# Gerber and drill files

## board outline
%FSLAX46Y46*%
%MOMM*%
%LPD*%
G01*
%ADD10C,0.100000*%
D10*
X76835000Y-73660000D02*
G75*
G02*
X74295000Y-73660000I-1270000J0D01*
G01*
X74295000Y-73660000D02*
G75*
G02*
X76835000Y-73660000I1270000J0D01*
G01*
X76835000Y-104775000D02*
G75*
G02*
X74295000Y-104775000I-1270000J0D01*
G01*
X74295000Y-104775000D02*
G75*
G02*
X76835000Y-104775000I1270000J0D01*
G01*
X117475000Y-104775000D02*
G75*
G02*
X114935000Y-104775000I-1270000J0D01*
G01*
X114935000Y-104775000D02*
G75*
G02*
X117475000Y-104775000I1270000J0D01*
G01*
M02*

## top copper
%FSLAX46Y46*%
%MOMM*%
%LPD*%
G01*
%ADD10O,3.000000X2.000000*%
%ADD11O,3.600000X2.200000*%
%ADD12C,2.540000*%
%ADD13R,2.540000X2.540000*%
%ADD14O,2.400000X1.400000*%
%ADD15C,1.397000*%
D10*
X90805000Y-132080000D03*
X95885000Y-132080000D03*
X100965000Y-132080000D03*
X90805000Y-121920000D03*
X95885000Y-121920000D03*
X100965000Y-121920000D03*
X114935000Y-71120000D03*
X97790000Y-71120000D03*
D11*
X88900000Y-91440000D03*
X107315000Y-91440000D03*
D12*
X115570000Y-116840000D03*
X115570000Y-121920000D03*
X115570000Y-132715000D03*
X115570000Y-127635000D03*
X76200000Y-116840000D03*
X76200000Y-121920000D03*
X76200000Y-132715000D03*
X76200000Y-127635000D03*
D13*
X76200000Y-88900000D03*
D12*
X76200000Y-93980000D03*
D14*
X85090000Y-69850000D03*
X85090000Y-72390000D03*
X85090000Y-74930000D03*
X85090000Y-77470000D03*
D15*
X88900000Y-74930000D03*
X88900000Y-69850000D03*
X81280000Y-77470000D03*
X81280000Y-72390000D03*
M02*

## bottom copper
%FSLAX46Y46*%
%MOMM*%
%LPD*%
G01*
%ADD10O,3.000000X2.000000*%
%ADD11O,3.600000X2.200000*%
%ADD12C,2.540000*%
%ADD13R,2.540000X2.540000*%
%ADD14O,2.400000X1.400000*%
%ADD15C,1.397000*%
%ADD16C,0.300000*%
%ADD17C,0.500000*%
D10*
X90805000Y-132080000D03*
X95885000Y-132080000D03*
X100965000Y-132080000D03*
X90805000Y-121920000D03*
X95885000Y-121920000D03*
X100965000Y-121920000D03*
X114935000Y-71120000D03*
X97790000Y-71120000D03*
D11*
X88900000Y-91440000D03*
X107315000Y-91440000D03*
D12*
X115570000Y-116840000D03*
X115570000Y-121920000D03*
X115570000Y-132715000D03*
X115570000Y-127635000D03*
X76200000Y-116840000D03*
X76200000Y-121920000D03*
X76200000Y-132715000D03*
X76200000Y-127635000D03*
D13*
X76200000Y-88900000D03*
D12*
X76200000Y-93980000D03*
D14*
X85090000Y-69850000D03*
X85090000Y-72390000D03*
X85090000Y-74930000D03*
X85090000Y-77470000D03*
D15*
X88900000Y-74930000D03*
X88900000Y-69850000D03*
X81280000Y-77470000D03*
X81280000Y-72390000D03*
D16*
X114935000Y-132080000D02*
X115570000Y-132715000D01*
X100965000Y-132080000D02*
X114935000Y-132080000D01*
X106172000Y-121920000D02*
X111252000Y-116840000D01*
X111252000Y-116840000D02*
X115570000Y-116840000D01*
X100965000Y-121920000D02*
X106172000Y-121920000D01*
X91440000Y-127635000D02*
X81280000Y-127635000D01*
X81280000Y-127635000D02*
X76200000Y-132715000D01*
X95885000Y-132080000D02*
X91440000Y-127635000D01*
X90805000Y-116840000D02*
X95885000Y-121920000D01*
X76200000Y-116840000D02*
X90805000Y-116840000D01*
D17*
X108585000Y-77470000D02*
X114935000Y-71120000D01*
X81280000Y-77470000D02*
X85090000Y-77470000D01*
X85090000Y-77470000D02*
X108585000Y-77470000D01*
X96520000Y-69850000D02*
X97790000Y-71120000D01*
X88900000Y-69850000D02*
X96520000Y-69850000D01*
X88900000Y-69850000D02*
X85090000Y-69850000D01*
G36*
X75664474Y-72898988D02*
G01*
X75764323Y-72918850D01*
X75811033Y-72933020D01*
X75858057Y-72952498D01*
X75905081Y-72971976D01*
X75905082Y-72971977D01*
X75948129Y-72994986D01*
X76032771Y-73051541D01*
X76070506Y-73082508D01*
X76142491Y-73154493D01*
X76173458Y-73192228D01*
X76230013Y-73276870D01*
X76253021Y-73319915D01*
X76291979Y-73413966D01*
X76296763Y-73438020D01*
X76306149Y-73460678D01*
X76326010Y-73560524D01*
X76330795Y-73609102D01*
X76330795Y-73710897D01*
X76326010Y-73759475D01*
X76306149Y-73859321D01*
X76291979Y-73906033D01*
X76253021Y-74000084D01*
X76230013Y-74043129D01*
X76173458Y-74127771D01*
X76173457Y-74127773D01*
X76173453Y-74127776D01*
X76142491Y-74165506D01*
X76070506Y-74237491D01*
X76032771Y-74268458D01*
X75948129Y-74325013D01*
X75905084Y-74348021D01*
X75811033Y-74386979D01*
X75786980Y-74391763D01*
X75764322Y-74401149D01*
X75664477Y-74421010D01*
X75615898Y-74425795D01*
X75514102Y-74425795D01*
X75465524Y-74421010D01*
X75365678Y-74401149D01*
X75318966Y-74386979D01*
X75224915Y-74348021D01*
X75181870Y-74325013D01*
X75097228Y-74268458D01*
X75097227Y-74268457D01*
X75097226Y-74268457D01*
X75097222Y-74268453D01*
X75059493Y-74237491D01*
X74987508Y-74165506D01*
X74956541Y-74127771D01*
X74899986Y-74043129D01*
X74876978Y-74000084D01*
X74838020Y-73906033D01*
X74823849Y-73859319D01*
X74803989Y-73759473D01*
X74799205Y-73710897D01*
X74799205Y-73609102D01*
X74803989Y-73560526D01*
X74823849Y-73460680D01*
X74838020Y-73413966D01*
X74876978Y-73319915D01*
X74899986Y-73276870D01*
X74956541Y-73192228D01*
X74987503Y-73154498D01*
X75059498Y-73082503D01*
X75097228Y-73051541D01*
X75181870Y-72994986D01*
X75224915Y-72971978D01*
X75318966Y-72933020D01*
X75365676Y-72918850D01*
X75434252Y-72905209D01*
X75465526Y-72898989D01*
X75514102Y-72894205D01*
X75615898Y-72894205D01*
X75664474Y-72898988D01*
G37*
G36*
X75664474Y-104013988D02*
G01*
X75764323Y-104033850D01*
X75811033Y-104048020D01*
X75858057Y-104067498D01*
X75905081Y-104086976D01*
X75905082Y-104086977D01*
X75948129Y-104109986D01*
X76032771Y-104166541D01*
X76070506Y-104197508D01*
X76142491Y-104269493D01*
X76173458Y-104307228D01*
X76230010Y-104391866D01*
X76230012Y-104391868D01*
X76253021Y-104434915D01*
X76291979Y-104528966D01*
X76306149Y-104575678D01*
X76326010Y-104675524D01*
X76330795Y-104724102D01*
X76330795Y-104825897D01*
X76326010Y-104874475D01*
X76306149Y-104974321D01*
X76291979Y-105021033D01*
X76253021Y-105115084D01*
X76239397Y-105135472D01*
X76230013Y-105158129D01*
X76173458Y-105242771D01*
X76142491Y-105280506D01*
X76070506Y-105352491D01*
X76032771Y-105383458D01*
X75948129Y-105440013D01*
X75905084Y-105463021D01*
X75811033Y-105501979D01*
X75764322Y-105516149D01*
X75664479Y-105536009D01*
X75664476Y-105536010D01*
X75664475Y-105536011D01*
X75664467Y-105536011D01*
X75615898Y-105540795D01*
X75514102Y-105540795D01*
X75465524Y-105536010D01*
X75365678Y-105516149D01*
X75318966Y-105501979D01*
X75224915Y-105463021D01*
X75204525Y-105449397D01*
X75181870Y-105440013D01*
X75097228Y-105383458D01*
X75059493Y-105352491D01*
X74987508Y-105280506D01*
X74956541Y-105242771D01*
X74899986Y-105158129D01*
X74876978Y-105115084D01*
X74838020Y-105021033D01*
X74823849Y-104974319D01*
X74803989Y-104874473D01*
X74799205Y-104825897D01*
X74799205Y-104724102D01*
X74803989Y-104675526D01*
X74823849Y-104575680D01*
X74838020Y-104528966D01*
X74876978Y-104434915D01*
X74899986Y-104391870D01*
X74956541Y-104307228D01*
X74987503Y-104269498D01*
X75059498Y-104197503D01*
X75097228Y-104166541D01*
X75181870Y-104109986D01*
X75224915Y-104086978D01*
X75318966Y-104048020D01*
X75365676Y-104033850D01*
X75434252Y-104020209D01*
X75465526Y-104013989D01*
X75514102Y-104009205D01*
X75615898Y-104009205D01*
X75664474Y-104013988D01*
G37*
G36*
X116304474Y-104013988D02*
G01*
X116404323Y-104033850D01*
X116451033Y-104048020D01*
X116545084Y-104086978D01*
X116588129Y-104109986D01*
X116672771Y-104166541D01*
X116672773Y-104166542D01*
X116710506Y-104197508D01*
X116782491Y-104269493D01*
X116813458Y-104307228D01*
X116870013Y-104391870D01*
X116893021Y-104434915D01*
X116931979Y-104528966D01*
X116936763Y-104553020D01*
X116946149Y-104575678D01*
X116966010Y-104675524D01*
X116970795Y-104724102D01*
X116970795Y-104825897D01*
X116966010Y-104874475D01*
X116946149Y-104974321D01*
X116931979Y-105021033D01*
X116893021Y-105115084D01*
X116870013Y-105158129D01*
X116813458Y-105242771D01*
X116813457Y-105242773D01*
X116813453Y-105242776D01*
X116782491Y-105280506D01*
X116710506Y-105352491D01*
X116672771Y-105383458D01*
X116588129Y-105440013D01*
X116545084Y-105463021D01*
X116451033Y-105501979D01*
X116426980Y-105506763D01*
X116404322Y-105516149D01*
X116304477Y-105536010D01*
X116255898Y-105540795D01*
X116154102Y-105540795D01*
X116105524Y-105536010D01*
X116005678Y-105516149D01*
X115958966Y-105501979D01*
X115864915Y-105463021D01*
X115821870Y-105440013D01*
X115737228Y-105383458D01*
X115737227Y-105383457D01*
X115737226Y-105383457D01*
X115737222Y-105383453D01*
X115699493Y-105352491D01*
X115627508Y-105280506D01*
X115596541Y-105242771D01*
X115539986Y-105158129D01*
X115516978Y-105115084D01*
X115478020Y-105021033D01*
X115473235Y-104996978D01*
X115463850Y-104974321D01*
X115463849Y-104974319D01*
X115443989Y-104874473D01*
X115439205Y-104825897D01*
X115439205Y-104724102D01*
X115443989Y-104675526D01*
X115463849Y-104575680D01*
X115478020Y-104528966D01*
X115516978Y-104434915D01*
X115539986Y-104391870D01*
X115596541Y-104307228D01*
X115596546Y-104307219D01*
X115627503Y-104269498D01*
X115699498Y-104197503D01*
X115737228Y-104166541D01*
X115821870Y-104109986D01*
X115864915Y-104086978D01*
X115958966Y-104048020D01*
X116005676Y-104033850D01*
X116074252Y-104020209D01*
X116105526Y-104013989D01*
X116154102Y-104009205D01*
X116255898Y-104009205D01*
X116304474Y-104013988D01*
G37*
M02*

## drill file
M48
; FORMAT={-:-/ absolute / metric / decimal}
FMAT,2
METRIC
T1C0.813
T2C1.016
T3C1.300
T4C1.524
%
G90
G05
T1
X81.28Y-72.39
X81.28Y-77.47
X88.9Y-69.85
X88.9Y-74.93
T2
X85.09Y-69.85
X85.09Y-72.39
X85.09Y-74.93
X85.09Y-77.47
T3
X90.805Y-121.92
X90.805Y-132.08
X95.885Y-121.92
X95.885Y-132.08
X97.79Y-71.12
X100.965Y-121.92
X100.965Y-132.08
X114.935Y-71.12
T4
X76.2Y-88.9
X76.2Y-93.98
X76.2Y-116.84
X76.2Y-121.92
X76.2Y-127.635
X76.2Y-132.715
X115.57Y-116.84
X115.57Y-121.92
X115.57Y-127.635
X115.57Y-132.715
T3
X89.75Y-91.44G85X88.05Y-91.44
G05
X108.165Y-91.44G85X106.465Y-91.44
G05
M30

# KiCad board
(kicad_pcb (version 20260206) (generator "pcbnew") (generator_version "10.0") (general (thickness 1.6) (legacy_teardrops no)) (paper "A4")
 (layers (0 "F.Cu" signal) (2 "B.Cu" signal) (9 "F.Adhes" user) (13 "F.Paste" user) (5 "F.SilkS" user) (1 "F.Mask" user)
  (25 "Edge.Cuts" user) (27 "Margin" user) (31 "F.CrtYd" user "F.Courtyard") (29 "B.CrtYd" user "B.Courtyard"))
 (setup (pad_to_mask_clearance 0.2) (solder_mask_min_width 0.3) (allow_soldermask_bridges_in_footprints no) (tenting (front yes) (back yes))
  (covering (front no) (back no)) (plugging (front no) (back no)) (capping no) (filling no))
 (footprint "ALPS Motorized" (layer "F.Cu") (at 95.885 96.52 180)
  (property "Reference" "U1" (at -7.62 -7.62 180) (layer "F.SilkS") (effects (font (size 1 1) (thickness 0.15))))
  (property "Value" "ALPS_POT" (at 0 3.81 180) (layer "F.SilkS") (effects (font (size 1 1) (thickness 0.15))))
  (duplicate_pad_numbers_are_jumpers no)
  (pad "1" thru_hole oval (at 5.08 -35.56 180) (size 3 2) (drill 1.3) (layers "*.Cu" "*.Mask" "F.SilkS") (remove_unused_layers no)
   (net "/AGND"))
  (pad "2" thru_hole oval (at 0 -35.56 180) (size 3 2) (drill 1.3) (layers "*.Cu" "*.Mask" "F.SilkS") (remove_unused_layers no)
   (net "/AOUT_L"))
  (pad "3" thru_hole oval (at -5.08 -35.56 180) (size 3 2) (drill 1.3) (layers "*.Cu" "*.Mask" "F.SilkS") (remove_unused_layers no)
   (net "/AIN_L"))
  (pad "4" thru_hole oval (at 5.08 -25.4 180) (size 3 2) (drill 1.3) (layers "*.Cu" "*.Mask" "F.SilkS") (remove_unused_layers no)
   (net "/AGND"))
  (pad "5" thru_hole oval (at 0 -25.4 180) (size 3 2) (drill 1.3) (layers "*.Cu" "*.Mask" "F.SilkS") (remove_unused_layers no)
   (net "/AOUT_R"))
  (pad "6" thru_hole oval (at -5.08 -25.4 180) (size 3 2) (drill 1.3) (layers "*.Cu" "*.Mask" "F.SilkS") (remove_unused_layers no)
   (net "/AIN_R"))
  (pad "7" thru_hole oval (at -19.05 25.4 180) (size 3 2) (drill 1.3) (layers "*.Cu" "*.Mask" "F.SilkS") (remove_unused_layers no)
   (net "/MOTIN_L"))
  (pad "8" thru_hole oval (at -1.905 25.4 180) (size 3 2) (drill 1.3) (layers "*.Cu" "*.Mask" "F.SilkS") (remove_unused_layers no)
   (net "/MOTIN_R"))
  (pad "9" thru_hole oval (at 6.985 5.08 180) (size 3.6 2.2) (drill oval 3 1.3) (layers "*.Cu" "*.Mask" "F.SilkS") (remove_unused_layers no)
   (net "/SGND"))
  (pad "10" thru_hole oval (at -11.43 5.08 180) (size 3.6 2.2) (drill oval 3 1.3) (layers "*.Cu" "*.Mask" "F.SilkS")
   (remove_unused_layers no) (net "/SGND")))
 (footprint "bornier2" (layer "F.Cu") (at 115.57 119.38 -90)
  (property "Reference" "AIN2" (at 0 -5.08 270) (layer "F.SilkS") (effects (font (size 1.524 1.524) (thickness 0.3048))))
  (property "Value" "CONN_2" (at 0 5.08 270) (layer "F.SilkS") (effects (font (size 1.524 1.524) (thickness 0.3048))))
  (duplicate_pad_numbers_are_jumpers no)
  (pad "1" thru_hole circle (at -2.54 0 270) (size 2.54 2.54) (drill 1.524) (layers "*.Cu" "*.Mask" "F.SilkS") (remove_unused_layers no)
   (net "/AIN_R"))
  (pad "2" thru_hole circle (at 2.54 0 270) (size 2.54 2.54) (drill 1.524) (layers "*.Cu" "*.Mask" "F.SilkS") (remove_unused_layers no)
   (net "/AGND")))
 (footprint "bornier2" (layer "F.Cu") (at 115.57 130.175 90)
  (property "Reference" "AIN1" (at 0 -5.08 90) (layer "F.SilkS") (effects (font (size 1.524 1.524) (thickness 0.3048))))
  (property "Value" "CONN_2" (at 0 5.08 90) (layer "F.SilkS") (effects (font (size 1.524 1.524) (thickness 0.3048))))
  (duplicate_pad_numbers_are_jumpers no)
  (pad "1" thru_hole circle (at -2.54 0 90) (size 2.54 2.54) (drill 1.524) (layers "*.Cu" "*.Mask" "F.SilkS") (remove_unused_layers no)
   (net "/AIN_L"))
  (pad "2" thru_hole circle (at 2.54 0 90) (size 2.54 2.54) (drill 1.524) (layers "*.Cu" "*.Mask" "F.SilkS") (remove_unused_layers no)
   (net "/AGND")))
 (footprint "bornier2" (layer "F.Cu") (at 76.2 119.38 -90)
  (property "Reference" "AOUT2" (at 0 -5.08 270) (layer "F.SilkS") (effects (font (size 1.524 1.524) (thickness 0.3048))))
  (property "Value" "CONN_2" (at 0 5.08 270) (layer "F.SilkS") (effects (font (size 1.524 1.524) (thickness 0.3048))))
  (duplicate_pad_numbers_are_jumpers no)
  (pad "1" thru_hole circle (at -2.54 0 270) (size 2.54 2.54) (drill 1.524) (layers "*.Cu" "*.Mask" "F.SilkS") (remove_unused_layers no)
   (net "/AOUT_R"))
  (pad "2" thru_hole circle (at 2.54 0 270) (size 2.54 2.54) (drill 1.524) (layers "*.Cu" "*.Mask" "F.SilkS") (remove_unused_layers no)
   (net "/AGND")))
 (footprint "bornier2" (layer "F.Cu") (at 76.2 130.175 90)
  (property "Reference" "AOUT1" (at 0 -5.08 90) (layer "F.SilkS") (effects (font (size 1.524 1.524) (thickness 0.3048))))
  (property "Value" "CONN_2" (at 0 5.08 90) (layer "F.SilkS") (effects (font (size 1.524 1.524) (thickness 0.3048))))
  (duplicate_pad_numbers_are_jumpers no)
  (pad "1" thru_hole circle (at -2.54 0 90) (size 2.54 2.54) (drill 1.524) (layers "*.Cu" "*.Mask" "F.SilkS") (remove_unused_layers no)
   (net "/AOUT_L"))
  (pad "2" thru_hole circle (at 2.54 0 90) (size 2.54 2.54) (drill 1.524) (layers "*.Cu" "*.Mask" "F.SilkS") (remove_unused_layers no)
   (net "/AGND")))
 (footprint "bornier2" (layer "F.Cu") (at 76.2 91.44 -90)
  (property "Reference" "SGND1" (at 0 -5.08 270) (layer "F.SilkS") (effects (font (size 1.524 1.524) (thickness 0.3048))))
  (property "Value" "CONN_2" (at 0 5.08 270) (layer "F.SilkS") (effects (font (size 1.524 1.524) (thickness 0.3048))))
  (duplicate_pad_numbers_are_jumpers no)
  (pad "1" thru_hole rect (at -2.54 0 270) (size 2.54 2.54) (drill 1.524) (layers "*.Cu" "*.Mask" "F.SilkS") (remove_unused_layers no)
   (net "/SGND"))
  (pad "2" thru_hole circle (at 2.54 0 270) (size 2.54 2.54) (drill 1.524) (layers "*.Cu" "*.Mask" "F.SilkS") (remove_unused_layers no)
   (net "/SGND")))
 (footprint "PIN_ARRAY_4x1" (layer "F.Cu") (at 85.09 73.66 -90)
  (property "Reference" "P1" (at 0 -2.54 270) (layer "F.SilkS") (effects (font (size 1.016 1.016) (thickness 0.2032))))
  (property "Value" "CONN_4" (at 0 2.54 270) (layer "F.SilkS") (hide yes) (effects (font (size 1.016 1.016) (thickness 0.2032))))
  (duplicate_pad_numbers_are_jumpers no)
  (pad "1" thru_hole oval (at -3.81 0 270) (size 1.4 2.4) (drill 1.016) (layers "*.Cu" "*.Mask" "F.SilkS") (remove_unused_layers no)
   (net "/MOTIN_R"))
  (pad "2" thru_hole oval (at -1.27 0 270) (size 1.4 2.4) (drill 1.016) (layers "*.Cu" "*.Mask" "F.SilkS") (remove_unused_layers no)
   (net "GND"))
  (pad "3" thru_hole oval (at 1.27 0 270) (size 1.4 2.4) (drill 1.016) (layers "*.Cu" "*.Mask" "F.SilkS") (remove_unused_layers no)
   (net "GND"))
  (pad "4" thru_hole oval (at 3.81 0 270) (size 1.4 2.4) (drill 1.016) (layers "*.Cu" "*.Mask" "F.SilkS") (remove_unused_layers no)
   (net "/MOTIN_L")))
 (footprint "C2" (layer "F.Cu") (at 88.9 72.39 90)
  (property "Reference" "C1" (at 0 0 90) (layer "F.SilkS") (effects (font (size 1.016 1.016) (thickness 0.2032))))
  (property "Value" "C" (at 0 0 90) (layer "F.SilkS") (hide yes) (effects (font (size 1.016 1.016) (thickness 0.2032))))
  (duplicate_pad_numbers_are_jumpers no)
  (pad "1" thru_hole circle (at -2.54 0 90) (size 1.397 1.397) (drill 0.8128) (layers "*.Cu" "*.Mask" "F.SilkS") (remove_unused_layers no)
   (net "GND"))
  (pad "2" thru_hole circle (at 2.54 0 90) (size 1.397 1.397) (drill 0.8128) (layers "*.Cu" "*.Mask" "F.SilkS") (remove_unused_layers no)
   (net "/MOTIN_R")))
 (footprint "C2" (layer "F.Cu") (at 81.28 74.93 90)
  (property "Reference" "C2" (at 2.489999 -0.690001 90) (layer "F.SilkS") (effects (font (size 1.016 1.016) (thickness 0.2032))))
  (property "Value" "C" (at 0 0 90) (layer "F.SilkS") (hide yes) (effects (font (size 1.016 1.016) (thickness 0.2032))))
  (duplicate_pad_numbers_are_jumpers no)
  (pad "1" thru_hole circle (at -2.54 0 90) (size 1.397 1.397) (drill 0.8128) (layers "*.Cu" "*.Mask" "F.SilkS") (remove_unused_layers no)
   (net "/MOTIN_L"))
  (pad "2" thru_hole circle (at 2.54 0 90) (size 1.397 1.397) (drill 0.8128) (layers "*.Cu" "*.Mask" "F.SilkS") (remove_unused_layers no)
   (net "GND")))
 (gr_circle (center 75.565 73.66) (end 76.835 73.66) (stroke (width 0.1) (type solid)) (fill no) (layer "Edge.Cuts"))
 (gr_circle (center 75.565 104.775) (end 76.835 104.775) (stroke (width 0.1) (type solid)) (fill no) (layer "Edge.Cuts"))
 (gr_circle (center 116.205 104.775) (end 117.475 104.775) (stroke (width 0.1) (type solid)) (fill no) (layer "Edge.Cuts"))
 (segment (start 114.935 132.08) (end 115.57 132.715) (width 0.3) (layer "B.Cu") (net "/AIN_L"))
 (segment (start 100.965 132.08) (end 114.935 132.08) (width 0.3) (layer "B.Cu") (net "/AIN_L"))
 (segment (start 106.172 121.92) (end 111.252 116.84) (width 0.3) (layer "B.Cu") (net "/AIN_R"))
 (segment (start 111.252 116.84) (end 115.57 116.84) (width 0.3) (layer "B.Cu") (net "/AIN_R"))
 (segment (start 100.965 121.92) (end 106.172 121.92) (width 0.3) (layer "B.Cu") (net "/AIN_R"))
 (segment (start 91.44 127.635) (end 81.28 127.635) (width 0.3) (layer "B.Cu") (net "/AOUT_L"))
 (segment (start 81.28 127.635) (end 76.2 132.715) (width 0.3) (layer "B.Cu") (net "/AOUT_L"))
 (segment (start 95.885 132.08) (end 91.44 127.635) (width 0.3) (layer "B.Cu") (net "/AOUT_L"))
 (segment (start 90.805 116.84) (end 95.885 121.92) (width 0.3) (layer "B.Cu") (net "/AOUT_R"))
 (segment (start 76.2 116.84) (end 90.805 116.84) (width 0.3) (layer "B.Cu") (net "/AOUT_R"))
 (segment (start 108.585 77.47) (end 114.935 71.12) (width 0.5) (layer "B.Cu") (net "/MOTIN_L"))
 (segment (start 81.28 77.47) (end 85.09 77.47) (width 0.5) (layer "B.Cu") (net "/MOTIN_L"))
 (segment (start 85.09 77.47) (end 108.585 77.47) (width 0.5) (layer "B.Cu") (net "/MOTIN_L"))
 (segment (start 96.52 69.85) (end 97.79 71.12) (width 0.5) (layer "B.Cu") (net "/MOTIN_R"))
 (segment (start 88.9 69.85) (end 96.52 69.85) (width 0.5) (layer "B.Cu") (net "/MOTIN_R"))
 (segment (start 88.9 69.85) (end 85.09 69.85) (width 0.5) (layer "B.Cu") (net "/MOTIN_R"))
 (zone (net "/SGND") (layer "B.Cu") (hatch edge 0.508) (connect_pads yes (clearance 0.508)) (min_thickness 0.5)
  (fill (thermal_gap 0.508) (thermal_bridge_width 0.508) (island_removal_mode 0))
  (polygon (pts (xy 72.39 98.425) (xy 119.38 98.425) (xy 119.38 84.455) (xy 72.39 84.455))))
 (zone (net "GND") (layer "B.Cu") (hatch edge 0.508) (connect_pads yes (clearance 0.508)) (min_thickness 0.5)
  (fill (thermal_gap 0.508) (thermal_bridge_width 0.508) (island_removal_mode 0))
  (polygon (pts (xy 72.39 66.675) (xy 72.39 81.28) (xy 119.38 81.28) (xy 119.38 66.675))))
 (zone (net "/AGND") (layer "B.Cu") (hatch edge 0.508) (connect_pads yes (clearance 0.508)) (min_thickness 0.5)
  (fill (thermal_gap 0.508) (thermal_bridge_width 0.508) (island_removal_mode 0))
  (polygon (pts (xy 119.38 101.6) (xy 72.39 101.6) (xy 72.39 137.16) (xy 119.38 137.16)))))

